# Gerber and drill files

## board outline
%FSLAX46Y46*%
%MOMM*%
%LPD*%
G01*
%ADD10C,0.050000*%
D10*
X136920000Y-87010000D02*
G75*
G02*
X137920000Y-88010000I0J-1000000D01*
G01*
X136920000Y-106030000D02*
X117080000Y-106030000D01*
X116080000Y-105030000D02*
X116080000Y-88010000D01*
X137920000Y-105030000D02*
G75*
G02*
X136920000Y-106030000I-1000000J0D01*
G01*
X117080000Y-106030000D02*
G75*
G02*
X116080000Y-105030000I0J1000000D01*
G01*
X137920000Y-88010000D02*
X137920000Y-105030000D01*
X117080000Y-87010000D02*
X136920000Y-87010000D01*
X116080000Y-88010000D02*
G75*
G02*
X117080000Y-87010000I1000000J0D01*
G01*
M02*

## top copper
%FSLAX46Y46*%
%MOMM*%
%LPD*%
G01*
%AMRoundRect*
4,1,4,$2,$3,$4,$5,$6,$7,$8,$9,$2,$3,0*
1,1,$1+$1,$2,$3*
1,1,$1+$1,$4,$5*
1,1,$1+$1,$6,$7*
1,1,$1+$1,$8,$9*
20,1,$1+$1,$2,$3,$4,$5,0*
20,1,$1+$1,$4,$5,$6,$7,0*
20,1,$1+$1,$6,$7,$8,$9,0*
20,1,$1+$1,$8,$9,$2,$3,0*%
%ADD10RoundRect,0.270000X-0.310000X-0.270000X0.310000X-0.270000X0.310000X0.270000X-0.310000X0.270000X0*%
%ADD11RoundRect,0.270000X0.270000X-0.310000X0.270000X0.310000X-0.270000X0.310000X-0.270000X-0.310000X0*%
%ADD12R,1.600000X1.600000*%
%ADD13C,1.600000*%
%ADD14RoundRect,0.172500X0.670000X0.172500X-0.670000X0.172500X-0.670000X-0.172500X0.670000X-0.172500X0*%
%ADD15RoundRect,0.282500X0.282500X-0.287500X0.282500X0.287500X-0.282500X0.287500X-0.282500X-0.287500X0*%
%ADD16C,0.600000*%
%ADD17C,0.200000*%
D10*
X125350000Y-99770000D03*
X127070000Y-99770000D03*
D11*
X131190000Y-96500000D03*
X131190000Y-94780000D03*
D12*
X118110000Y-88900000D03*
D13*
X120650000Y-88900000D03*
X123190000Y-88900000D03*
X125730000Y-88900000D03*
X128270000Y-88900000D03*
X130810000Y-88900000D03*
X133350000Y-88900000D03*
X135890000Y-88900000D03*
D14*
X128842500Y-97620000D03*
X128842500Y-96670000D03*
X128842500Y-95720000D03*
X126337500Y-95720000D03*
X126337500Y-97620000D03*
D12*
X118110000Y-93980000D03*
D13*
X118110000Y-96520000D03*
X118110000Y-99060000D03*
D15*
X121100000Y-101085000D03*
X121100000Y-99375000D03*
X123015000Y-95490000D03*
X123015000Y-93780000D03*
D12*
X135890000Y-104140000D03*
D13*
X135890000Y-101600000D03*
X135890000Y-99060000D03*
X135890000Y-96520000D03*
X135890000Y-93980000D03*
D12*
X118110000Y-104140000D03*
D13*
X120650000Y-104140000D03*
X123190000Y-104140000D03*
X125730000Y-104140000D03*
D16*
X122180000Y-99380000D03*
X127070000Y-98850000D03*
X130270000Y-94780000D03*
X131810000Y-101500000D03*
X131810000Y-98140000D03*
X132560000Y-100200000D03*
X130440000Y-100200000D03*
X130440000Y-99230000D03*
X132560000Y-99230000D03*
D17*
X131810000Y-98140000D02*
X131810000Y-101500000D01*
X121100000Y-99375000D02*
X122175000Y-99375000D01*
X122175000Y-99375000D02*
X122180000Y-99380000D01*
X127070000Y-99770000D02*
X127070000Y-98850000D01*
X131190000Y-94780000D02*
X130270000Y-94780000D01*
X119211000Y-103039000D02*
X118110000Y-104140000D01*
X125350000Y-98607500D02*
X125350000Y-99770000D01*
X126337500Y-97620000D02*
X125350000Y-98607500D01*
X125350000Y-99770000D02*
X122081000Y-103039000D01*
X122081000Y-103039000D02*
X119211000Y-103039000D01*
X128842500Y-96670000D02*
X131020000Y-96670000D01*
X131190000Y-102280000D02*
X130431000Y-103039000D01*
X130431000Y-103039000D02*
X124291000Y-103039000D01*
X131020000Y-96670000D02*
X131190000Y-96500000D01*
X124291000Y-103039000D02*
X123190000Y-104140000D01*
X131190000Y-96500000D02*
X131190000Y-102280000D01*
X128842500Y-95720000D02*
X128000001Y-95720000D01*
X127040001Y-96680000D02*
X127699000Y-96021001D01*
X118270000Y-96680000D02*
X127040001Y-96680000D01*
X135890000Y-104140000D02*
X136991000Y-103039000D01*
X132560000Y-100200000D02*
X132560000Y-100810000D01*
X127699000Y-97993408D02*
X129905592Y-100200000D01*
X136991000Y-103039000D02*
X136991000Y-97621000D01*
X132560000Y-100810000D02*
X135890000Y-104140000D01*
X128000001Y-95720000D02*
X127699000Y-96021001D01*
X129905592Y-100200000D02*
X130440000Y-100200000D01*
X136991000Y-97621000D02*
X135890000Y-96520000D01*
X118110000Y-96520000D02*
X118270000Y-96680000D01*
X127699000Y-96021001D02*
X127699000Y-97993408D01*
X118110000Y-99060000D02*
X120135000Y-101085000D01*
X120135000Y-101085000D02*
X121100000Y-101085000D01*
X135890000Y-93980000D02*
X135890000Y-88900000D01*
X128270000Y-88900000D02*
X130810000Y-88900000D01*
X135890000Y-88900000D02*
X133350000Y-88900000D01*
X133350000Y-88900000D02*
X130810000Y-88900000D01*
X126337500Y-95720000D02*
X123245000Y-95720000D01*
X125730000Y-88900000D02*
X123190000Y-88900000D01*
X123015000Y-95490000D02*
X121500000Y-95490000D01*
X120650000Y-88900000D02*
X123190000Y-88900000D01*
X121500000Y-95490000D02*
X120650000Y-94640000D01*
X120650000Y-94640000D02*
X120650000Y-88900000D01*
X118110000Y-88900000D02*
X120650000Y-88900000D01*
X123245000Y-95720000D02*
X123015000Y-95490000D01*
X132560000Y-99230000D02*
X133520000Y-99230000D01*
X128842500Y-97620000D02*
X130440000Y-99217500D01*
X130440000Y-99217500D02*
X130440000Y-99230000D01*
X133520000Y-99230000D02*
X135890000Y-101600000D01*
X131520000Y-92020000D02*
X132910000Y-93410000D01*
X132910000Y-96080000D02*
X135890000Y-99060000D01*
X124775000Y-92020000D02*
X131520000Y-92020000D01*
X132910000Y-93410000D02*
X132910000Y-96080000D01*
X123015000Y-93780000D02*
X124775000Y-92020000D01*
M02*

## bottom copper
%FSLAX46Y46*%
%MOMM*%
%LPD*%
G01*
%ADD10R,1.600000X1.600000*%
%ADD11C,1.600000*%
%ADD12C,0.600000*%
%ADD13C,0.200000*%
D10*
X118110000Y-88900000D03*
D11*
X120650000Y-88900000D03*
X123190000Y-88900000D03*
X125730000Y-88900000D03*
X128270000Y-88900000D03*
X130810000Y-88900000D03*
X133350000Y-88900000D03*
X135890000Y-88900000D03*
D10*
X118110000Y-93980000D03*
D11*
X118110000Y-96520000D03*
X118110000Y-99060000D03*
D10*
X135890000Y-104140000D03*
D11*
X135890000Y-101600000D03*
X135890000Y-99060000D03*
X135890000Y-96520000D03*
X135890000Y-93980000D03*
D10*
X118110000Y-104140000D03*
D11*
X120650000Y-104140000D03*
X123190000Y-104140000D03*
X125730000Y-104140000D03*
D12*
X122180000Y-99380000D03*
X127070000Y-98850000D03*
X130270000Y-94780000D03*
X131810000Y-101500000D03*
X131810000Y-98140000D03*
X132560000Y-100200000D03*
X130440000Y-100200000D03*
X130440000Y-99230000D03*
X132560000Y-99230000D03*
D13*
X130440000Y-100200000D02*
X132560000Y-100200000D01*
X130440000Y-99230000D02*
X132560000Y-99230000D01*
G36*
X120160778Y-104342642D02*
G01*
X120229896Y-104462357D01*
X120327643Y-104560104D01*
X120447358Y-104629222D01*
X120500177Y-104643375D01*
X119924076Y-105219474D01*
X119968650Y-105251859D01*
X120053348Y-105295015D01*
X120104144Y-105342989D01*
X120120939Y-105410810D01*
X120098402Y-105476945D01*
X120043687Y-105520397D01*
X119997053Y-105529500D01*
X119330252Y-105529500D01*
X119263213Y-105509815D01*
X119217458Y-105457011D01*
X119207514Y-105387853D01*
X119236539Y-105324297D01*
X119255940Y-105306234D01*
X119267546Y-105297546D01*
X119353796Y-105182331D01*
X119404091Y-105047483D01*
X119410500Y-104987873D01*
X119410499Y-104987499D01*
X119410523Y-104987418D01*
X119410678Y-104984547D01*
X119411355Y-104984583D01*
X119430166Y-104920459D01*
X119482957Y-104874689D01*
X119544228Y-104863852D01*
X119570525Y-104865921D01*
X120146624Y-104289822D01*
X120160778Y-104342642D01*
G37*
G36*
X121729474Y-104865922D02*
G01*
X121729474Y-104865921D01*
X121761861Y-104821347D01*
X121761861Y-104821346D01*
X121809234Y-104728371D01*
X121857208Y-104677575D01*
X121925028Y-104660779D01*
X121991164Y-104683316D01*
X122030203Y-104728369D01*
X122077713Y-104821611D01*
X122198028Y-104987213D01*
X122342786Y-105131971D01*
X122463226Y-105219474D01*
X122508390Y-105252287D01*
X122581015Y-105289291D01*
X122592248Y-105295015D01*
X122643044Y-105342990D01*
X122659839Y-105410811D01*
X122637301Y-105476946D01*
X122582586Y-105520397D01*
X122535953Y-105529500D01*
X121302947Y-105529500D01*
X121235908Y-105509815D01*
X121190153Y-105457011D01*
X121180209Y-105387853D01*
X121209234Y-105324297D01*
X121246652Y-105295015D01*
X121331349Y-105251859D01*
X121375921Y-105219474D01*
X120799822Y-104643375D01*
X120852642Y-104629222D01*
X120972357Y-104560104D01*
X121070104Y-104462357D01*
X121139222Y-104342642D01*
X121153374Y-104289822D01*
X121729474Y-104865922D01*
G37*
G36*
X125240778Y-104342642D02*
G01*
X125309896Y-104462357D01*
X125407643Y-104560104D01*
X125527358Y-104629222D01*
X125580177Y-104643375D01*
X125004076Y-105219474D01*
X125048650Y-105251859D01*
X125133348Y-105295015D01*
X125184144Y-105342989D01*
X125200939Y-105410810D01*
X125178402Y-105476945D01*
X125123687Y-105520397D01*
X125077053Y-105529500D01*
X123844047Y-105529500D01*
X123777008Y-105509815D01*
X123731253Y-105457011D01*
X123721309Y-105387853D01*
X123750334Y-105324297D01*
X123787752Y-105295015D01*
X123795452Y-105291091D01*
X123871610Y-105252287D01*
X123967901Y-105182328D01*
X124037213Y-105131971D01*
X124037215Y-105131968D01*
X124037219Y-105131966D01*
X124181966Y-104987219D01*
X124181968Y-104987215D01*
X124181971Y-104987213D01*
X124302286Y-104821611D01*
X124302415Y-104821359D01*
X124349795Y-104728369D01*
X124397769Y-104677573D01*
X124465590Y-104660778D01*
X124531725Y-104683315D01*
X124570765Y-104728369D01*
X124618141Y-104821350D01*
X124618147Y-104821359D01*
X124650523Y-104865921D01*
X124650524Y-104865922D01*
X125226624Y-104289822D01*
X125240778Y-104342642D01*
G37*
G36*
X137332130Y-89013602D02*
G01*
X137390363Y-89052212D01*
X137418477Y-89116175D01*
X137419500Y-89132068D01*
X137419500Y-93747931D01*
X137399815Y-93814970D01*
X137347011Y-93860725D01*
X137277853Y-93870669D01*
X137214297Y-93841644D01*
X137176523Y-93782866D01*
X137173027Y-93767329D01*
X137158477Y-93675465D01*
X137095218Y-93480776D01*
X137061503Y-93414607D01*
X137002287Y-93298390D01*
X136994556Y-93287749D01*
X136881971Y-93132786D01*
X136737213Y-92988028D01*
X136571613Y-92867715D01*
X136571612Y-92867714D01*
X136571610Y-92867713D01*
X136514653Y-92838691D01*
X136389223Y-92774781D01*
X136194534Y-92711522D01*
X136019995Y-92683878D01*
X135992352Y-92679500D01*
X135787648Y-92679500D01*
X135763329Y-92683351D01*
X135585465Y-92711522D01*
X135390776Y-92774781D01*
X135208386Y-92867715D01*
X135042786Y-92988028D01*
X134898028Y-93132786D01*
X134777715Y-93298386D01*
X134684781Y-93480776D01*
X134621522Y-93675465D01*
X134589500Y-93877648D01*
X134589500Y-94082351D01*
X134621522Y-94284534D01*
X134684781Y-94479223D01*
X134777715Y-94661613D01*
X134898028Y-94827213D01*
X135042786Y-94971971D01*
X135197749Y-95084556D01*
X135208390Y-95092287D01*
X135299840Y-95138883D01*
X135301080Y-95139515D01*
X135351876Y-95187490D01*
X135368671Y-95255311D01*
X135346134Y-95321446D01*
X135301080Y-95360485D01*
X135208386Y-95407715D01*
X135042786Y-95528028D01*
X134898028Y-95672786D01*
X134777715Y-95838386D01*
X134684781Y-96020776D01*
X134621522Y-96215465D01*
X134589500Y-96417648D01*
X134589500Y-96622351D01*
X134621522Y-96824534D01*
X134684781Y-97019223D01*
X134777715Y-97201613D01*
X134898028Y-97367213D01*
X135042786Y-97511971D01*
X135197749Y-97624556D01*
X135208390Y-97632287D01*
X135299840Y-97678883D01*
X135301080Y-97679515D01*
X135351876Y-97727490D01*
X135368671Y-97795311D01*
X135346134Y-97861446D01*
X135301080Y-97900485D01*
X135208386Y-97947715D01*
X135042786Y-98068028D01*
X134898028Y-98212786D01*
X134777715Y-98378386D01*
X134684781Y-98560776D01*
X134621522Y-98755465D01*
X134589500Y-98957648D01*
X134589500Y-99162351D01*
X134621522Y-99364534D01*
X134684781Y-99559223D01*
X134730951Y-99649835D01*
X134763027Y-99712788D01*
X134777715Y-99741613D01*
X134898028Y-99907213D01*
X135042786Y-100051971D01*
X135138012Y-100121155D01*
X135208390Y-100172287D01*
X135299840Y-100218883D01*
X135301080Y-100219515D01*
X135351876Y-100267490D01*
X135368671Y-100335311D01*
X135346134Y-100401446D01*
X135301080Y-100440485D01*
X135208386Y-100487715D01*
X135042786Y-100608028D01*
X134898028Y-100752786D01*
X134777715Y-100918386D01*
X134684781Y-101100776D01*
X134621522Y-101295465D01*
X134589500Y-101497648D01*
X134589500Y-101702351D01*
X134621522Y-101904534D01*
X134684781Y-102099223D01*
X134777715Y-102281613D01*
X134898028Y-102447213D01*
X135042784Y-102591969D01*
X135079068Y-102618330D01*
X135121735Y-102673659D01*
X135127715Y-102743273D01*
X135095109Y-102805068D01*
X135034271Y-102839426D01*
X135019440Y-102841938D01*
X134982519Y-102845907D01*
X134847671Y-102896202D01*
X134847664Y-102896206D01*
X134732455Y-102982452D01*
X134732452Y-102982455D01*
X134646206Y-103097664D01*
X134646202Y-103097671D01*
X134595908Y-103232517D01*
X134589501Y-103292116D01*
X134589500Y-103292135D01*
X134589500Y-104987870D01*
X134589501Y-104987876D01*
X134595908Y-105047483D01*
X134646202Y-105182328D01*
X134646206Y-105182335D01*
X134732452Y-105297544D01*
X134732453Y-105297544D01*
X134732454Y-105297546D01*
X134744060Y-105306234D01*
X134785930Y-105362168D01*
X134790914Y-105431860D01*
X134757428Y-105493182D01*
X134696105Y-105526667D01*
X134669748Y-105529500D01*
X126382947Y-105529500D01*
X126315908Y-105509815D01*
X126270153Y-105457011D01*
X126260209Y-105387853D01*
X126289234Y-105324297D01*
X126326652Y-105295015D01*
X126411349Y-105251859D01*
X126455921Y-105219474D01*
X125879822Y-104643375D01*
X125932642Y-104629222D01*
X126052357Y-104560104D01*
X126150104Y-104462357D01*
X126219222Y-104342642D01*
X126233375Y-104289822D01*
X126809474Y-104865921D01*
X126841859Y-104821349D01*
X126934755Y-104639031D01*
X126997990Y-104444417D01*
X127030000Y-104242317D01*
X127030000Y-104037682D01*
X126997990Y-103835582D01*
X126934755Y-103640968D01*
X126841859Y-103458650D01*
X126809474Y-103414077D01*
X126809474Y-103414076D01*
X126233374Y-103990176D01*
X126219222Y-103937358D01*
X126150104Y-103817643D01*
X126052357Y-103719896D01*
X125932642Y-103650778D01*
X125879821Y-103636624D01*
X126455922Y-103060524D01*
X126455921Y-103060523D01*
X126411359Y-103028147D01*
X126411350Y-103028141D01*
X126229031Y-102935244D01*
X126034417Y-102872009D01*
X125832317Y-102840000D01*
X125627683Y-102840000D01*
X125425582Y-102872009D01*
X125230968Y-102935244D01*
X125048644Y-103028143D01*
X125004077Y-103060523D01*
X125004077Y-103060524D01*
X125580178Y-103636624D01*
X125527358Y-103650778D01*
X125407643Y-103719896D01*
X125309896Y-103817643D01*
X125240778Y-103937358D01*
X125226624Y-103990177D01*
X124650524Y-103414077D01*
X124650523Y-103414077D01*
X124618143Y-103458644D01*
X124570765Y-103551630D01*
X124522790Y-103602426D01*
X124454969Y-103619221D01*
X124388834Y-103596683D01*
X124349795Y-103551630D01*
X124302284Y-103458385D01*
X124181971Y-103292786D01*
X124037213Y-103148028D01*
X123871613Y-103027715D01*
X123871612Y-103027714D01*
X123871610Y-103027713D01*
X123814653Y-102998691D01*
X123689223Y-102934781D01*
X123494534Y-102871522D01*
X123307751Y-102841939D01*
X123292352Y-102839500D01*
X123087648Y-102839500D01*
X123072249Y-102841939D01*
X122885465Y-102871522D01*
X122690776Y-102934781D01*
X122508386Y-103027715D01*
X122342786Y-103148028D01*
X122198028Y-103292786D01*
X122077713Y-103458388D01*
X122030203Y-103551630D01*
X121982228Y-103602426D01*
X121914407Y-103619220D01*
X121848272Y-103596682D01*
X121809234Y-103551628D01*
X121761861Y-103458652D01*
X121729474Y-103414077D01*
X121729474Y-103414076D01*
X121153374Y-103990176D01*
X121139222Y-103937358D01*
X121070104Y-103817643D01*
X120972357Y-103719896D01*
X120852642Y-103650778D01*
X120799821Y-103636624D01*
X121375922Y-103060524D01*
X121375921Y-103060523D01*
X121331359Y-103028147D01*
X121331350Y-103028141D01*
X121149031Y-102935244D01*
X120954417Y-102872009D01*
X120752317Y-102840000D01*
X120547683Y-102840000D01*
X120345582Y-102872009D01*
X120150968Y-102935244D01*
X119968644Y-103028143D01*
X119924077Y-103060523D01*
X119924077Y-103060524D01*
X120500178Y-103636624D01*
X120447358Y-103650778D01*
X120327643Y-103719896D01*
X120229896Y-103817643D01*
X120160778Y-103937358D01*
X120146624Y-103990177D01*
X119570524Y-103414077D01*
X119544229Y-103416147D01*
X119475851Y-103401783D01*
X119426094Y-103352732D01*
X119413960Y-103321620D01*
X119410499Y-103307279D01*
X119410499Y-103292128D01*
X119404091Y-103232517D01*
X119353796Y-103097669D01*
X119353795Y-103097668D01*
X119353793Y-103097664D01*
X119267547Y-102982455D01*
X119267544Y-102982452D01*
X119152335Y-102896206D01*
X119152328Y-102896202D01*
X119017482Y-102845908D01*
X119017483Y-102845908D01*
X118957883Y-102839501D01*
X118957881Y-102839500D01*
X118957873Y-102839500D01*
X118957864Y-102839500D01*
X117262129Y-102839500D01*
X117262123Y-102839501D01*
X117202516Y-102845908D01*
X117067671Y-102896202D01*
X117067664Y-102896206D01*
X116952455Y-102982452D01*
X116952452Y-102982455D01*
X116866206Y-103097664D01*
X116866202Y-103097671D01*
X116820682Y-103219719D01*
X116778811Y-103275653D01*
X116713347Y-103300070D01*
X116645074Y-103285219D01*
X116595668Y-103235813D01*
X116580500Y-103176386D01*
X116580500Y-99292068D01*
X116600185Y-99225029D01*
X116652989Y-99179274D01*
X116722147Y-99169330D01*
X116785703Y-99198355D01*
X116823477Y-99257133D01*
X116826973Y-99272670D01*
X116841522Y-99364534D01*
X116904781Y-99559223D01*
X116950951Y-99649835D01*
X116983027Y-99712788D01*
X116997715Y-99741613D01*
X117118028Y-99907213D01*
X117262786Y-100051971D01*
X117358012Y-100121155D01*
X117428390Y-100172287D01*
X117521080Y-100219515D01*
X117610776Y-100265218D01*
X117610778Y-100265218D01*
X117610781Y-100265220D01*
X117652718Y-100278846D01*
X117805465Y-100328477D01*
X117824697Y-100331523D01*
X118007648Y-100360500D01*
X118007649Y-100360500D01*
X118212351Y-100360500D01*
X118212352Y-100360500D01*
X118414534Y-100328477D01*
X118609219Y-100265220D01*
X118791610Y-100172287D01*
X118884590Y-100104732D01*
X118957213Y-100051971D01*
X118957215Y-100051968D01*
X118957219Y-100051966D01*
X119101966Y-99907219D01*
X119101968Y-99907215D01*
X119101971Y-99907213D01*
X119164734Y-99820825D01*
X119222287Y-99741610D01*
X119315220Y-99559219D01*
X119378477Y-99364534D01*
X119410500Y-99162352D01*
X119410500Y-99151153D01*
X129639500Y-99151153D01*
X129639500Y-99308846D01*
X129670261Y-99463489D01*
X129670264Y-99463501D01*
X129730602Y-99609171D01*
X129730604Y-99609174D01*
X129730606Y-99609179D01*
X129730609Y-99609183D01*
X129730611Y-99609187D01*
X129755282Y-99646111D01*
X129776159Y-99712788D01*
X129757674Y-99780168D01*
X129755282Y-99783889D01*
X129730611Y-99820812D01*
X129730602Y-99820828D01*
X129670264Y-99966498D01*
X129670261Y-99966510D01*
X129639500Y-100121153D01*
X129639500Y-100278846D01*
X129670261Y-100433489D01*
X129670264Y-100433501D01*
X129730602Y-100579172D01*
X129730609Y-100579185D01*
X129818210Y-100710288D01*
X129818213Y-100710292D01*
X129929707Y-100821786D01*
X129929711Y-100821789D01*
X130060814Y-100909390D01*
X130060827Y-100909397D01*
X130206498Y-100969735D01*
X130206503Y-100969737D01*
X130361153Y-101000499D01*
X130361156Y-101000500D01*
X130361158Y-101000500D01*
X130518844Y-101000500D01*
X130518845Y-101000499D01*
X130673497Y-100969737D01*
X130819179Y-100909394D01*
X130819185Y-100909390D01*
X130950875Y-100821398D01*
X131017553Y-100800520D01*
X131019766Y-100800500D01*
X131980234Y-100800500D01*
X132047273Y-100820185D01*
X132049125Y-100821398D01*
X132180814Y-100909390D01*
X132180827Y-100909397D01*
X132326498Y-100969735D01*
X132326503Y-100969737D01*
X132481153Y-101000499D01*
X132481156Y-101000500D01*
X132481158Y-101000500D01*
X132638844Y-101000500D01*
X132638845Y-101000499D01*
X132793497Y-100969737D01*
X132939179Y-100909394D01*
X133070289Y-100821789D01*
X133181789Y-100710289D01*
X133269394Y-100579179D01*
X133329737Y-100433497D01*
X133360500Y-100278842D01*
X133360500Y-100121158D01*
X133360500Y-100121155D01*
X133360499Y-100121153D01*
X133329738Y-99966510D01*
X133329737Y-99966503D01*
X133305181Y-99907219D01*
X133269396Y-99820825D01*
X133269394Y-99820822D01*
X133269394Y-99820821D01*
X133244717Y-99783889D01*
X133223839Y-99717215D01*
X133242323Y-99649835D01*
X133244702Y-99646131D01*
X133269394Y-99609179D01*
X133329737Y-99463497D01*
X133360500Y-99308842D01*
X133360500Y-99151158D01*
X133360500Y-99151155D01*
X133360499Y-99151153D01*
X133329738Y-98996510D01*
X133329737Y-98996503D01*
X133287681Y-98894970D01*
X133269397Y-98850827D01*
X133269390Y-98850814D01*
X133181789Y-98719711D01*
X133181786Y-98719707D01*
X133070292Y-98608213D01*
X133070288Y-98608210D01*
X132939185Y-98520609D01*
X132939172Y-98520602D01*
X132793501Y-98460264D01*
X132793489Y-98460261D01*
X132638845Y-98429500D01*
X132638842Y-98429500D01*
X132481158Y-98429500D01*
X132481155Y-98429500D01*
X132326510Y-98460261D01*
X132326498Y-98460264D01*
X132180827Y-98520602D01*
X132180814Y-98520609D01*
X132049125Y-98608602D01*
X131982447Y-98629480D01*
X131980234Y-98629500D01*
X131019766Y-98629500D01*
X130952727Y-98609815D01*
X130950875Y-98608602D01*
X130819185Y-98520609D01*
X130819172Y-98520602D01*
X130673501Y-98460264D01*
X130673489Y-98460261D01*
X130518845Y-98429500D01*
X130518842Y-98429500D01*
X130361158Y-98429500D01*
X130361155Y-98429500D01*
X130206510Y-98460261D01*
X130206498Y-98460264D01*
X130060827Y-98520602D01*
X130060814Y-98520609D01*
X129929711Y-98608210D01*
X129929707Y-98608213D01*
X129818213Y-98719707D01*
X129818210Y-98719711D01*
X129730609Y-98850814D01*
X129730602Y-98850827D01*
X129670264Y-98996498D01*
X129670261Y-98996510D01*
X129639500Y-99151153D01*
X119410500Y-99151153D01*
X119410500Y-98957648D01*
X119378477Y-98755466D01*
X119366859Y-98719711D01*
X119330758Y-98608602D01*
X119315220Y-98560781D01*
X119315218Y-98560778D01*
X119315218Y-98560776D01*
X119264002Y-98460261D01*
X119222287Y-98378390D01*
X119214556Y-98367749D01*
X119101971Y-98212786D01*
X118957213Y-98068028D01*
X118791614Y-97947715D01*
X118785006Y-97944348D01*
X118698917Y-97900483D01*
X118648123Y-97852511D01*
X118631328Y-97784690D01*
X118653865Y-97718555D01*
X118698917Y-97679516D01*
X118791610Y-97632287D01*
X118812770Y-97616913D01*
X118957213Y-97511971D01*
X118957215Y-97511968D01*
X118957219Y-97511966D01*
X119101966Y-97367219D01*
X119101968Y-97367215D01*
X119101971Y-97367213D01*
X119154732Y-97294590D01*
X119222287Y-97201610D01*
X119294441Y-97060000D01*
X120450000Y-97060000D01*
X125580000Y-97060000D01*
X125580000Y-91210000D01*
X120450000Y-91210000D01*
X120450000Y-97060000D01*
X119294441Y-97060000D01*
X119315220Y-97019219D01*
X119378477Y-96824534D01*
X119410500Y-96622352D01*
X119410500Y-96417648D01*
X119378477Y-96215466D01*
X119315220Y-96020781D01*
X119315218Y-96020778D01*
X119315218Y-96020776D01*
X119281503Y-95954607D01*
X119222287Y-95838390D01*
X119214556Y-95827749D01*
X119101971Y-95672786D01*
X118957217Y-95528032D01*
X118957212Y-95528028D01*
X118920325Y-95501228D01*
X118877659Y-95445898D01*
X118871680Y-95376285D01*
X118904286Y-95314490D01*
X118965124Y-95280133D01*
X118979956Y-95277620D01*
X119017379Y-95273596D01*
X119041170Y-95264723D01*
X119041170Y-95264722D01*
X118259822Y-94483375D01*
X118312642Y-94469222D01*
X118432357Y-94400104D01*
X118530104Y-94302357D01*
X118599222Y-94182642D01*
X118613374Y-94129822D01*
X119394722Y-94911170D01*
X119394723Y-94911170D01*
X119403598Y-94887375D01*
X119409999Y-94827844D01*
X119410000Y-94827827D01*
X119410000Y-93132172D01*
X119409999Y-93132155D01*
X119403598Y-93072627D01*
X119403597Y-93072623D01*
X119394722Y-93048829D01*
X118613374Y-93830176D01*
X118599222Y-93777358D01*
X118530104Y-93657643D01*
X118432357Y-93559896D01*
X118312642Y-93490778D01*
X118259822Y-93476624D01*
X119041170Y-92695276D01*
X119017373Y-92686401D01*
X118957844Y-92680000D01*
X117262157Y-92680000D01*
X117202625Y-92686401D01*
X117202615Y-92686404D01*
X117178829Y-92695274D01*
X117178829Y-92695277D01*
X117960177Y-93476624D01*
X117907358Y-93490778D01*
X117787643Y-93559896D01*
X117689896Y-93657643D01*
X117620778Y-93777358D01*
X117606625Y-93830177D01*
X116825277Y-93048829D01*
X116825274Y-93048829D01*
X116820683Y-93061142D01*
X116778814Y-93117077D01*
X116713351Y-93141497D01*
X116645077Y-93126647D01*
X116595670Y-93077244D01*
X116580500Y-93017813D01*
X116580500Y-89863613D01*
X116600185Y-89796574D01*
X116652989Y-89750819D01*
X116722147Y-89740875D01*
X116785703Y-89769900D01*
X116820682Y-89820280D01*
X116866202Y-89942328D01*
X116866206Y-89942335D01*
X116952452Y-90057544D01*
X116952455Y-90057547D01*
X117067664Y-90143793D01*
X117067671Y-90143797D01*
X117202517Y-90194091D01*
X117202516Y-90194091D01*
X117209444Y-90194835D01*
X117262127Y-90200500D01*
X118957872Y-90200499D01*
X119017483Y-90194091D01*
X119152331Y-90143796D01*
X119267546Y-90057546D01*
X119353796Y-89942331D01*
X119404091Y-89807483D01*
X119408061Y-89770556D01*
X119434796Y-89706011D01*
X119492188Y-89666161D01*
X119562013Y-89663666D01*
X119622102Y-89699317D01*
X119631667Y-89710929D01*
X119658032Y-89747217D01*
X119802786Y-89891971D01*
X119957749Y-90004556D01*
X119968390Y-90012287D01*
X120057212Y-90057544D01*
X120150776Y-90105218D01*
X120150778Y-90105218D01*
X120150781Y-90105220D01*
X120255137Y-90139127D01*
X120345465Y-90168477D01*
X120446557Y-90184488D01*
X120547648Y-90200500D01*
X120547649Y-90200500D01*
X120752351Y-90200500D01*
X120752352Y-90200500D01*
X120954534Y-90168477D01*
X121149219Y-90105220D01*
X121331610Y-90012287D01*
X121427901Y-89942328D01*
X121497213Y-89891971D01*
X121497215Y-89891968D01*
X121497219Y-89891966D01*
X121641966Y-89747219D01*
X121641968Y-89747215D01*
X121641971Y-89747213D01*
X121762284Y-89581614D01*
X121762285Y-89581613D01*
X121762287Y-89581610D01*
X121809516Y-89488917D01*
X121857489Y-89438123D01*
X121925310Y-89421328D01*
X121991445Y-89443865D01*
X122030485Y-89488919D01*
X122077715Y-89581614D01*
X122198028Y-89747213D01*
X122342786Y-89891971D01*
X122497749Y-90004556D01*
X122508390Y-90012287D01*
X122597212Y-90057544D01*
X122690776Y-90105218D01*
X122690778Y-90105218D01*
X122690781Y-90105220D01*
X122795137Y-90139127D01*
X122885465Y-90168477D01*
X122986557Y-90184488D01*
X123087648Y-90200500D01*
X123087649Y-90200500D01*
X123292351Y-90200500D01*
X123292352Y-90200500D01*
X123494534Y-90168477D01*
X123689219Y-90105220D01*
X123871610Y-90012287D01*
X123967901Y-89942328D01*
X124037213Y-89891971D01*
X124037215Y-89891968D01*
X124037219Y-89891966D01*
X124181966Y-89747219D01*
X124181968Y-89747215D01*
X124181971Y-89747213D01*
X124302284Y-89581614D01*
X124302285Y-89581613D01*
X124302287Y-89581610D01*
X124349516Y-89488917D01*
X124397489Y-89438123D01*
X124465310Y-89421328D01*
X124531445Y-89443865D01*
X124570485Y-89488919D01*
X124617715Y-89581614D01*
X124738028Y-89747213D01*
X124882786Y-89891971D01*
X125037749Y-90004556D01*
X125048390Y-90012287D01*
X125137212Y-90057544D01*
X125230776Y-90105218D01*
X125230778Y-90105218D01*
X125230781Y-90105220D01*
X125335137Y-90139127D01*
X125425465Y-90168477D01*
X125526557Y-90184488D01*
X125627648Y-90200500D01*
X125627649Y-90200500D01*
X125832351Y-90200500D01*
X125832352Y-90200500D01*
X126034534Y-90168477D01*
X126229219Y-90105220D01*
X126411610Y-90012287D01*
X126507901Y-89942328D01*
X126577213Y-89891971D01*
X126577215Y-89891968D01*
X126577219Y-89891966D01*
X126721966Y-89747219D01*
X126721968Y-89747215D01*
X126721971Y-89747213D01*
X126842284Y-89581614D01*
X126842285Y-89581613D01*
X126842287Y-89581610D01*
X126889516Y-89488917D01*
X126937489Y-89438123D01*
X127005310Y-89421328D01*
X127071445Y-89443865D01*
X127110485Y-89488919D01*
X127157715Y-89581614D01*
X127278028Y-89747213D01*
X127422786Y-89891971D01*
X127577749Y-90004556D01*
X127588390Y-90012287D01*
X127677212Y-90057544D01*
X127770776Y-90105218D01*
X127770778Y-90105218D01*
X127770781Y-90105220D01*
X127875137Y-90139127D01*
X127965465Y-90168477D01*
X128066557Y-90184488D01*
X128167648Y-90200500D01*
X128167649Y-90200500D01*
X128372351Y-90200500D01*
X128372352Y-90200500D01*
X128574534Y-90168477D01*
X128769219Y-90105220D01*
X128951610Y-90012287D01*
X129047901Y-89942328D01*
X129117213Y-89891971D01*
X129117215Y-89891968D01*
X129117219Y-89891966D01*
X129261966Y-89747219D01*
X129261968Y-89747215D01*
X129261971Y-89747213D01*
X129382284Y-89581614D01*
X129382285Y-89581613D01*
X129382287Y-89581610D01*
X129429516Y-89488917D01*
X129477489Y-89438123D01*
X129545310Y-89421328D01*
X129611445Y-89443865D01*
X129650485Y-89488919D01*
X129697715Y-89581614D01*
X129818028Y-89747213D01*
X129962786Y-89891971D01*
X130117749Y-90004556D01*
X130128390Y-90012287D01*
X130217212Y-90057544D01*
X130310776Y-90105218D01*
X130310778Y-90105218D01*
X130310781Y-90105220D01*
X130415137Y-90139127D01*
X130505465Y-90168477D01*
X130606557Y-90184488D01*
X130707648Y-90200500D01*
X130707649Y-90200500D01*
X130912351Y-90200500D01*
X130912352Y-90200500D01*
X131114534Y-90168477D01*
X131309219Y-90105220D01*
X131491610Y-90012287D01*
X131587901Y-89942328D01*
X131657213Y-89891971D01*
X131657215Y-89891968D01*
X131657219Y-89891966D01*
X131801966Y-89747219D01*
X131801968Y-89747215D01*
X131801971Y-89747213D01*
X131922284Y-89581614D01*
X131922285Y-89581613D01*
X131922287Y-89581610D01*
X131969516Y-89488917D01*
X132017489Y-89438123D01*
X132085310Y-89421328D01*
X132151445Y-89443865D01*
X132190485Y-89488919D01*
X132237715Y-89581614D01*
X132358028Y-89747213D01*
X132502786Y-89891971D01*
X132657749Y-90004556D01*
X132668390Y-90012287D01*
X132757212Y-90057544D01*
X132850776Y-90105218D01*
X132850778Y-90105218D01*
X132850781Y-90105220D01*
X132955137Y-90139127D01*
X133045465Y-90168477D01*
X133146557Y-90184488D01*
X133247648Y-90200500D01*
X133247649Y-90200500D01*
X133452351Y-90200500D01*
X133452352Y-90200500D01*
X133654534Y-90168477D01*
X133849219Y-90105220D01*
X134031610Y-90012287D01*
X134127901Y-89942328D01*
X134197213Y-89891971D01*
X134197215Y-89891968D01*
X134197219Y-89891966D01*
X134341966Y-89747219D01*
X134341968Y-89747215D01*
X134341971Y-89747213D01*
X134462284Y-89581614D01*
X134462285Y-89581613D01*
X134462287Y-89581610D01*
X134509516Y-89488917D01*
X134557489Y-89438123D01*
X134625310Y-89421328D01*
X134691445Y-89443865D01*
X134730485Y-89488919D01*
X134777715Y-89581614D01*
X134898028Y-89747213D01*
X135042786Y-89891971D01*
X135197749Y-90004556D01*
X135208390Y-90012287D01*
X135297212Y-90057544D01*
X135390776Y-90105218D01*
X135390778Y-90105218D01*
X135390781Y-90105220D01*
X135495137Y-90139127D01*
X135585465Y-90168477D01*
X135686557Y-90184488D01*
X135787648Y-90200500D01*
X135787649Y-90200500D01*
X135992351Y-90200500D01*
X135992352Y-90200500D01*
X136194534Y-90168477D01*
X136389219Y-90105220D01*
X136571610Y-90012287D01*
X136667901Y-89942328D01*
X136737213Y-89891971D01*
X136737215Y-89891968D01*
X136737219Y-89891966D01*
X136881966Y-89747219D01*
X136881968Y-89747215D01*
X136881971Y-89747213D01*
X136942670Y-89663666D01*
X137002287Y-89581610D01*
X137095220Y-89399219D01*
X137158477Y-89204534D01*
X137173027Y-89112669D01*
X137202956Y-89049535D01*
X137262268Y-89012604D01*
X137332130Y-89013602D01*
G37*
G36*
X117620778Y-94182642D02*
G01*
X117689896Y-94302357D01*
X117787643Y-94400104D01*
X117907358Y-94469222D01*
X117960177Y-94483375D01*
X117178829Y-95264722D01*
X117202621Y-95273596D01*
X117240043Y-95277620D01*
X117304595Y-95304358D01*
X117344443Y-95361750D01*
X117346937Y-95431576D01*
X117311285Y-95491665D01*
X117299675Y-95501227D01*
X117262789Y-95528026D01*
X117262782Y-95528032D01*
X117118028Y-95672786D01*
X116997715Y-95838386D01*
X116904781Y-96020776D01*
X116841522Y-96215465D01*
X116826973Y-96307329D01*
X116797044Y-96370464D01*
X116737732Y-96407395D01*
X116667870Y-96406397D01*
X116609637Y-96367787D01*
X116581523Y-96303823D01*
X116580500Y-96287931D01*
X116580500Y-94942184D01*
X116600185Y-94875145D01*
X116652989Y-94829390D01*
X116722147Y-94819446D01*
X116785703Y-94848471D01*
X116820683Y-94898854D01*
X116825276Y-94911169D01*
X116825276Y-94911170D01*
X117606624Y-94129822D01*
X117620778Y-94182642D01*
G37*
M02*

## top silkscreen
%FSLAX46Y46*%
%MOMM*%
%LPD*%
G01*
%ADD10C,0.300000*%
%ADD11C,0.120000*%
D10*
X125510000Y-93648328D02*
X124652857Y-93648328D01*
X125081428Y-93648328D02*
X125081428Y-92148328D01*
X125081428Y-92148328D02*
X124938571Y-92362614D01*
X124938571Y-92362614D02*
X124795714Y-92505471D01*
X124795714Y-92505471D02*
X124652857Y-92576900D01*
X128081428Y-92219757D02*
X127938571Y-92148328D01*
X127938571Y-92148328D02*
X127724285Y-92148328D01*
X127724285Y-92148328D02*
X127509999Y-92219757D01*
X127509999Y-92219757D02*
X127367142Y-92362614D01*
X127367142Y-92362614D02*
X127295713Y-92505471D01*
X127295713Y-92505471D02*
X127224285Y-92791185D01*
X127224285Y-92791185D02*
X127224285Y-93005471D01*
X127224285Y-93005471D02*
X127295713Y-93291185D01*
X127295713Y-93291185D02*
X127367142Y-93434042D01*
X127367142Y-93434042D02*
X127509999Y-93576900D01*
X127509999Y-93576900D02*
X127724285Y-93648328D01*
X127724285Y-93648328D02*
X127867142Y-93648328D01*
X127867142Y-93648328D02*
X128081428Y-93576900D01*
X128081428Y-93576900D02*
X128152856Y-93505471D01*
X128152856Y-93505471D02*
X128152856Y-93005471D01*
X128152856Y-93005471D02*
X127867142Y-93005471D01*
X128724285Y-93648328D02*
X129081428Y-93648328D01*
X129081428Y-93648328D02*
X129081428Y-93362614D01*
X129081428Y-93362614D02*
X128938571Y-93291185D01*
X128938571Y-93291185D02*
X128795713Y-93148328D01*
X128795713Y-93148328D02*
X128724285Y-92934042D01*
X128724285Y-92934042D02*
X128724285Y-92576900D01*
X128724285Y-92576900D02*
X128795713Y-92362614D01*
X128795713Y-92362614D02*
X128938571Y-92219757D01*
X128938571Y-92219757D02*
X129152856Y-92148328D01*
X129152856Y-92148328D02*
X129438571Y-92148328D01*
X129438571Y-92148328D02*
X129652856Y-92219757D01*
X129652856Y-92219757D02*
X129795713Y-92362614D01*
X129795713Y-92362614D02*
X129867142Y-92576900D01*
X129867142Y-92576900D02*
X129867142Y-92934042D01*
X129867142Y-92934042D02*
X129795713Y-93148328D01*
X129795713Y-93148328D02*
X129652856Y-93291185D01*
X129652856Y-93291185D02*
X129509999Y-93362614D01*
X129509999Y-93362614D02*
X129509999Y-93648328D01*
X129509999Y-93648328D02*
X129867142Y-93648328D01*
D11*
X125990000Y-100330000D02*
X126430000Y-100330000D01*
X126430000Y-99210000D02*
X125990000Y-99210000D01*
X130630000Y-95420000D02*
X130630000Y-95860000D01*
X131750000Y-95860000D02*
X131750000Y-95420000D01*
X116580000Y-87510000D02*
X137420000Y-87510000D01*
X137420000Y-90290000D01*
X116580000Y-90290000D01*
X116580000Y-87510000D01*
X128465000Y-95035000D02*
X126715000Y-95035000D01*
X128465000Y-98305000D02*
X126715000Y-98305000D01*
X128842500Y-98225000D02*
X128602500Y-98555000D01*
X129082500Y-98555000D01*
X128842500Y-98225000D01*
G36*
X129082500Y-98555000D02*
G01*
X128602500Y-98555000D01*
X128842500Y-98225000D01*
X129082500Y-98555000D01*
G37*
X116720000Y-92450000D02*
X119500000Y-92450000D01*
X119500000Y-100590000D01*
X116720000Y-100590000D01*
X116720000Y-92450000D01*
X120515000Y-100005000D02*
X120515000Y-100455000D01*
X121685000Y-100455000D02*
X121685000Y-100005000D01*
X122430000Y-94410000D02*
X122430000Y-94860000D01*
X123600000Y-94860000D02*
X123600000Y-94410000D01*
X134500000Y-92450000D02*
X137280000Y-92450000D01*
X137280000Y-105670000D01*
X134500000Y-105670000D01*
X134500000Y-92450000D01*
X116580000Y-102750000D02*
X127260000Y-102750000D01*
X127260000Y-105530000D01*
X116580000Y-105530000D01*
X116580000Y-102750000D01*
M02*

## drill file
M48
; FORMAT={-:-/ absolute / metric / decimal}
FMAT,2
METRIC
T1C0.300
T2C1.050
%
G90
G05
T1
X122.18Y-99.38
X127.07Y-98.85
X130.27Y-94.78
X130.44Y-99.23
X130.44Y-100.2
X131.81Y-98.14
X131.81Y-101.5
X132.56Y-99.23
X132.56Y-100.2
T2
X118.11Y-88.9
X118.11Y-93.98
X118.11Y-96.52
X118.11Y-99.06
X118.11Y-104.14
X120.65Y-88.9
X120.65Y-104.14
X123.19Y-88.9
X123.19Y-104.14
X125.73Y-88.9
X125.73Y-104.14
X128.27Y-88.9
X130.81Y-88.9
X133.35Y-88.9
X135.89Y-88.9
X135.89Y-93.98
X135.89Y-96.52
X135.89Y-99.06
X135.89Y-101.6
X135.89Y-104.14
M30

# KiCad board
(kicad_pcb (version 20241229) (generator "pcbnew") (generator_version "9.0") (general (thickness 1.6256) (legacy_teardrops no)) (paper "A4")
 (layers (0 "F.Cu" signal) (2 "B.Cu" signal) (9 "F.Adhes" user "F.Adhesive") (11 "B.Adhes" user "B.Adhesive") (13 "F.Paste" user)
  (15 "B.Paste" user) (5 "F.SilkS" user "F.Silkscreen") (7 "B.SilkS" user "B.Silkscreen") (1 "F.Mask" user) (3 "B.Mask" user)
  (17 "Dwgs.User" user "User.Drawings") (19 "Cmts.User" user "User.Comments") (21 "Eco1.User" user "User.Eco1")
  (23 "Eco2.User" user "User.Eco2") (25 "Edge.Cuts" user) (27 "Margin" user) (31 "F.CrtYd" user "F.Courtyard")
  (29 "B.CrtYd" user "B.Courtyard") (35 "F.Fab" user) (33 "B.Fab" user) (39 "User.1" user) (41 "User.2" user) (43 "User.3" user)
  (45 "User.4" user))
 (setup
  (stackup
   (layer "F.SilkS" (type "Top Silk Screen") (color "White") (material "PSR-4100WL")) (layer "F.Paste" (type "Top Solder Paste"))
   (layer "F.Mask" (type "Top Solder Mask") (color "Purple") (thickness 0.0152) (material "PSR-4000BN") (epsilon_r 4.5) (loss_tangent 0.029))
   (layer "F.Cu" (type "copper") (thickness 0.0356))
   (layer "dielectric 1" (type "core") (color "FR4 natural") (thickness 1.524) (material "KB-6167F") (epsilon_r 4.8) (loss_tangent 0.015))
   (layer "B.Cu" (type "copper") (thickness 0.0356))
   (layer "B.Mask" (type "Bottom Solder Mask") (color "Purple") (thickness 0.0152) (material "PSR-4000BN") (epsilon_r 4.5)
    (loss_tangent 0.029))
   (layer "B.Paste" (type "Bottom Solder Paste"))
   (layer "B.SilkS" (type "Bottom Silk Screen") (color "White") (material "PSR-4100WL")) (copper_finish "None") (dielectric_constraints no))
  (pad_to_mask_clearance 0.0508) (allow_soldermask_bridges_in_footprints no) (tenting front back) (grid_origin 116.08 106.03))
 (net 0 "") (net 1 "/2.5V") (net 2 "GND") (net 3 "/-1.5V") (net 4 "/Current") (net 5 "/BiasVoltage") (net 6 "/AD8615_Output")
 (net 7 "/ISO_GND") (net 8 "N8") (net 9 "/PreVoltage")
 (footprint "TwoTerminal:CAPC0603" (layer "F.Cu") (at 126.21 99.77)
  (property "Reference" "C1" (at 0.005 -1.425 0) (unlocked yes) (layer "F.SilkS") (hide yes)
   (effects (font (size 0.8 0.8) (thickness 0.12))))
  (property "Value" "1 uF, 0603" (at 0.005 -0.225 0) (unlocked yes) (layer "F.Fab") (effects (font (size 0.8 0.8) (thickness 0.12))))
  (fp_line (start -0.22 0.56) (end 0.22 0.56) (stroke (width 0.12) (type default)) (layer "F.SilkS"))
  (fp_line (start 0.22 -0.56) (end -0.22 -0.56) (stroke (width 0.12) (type default)) (layer "F.SilkS"))
  (pad "1" smd roundrect (at -0.86 0) (size 1.16 1.08) (layers "F.Cu" "F.Mask" "F.Paste") (roundrect_rratio 0.25) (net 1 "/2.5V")
   (thermal_bridge_angle 45))
  (pad "2" smd roundrect (at 0.86 0) (size 1.16 1.08) (layers "F.Cu" "F.Mask" "F.Paste") (roundrect_rratio 0.25) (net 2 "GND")
   (thermal_bridge_angle 45)))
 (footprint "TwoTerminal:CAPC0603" (layer "F.Cu") (at 131.19 95.64 90)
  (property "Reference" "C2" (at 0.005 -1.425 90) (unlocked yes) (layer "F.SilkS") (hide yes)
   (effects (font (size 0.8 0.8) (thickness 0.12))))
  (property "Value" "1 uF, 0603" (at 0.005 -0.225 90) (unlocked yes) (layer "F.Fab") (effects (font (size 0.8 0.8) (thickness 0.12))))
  (fp_line (start 0.22 -0.56) (end -0.22 -0.56) (stroke (width 0.12) (type default)) (layer "F.SilkS"))
  (fp_line (start -0.22 0.56) (end 0.22 0.56) (stroke (width 0.12) (type default)) (layer "F.SilkS"))
  (pad "1" smd roundrect (at -0.86 0 90) (size 1.16 1.08) (layers "F.Cu" "F.Mask" "F.Paste") (roundrect_rratio 0.25) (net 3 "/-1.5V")
   (thermal_bridge_angle 45))
  (pad "2" smd roundrect (at 0.86 0 90) (size 1.16 1.08) (layers "F.Cu" "F.Mask" "F.Paste") (roundrect_rratio 0.25) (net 2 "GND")
   (thermal_bridge_angle 45)))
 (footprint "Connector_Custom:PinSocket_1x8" (layer "F.Cu") (at 127 88.9 90)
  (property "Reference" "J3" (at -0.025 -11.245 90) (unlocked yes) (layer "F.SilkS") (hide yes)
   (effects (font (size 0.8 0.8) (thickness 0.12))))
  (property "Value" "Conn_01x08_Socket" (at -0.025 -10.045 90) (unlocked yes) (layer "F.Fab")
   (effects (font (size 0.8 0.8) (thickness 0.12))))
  (fp_rect (start -1.39 -10.42) (end 1.39 10.42) (stroke (width 0.12) (type default)) (fill no) (layer "F.SilkS"))
  (pad "1" thru_hole rect (at 0 -8.89 90) (size 1.6 1.6) (drill 1.05) (layers "*.Cu" "*.Mask") (remove_unused_layers no) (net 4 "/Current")
   (thermal_bridge_angle 45))
  (pad "2" thru_hole circle (at 0 -6.35 90) (size 1.6 1.6) (drill 1.05) (layers "*.Cu" "*.Mask") (remove_unused_layers no)
   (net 4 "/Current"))
  (pad "3" thru_hole circle (at 0 -3.81 90) (size 1.6 1.6) (drill 1.05) (layers "*.Cu" "*.Mask") (remove_unused_layers no)
   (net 4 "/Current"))
  (pad "4" thru_hole circle (at 0 -1.27 90) (size 1.6 1.6) (drill 1.05) (layers "*.Cu" "*.Mask") (remove_unused_layers no)
   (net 4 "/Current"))
  (pad "5" thru_hole circle (at 0 1.27 90) (size 1.6 1.6) (drill 1.05) (layers "*.Cu" "*.Mask") (remove_unused_layers no)
   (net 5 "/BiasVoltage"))
  (pad "6" thru_hole circle (at 0 3.81 90) (size 1.6 1.6) (drill 1.05) (layers "*.Cu" "*.Mask") (remove_unused_layers no)
   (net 5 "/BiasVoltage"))
  (pad "7" thru_hole circle (at 0 6.35 90) (size 1.6 1.6) (drill 1.05) (layers "*.Cu" "*.Mask") (remove_unused_layers no)
   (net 5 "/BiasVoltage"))
  (pad "8" thru_hole circle (at 0 8.89 90) (size 1.6 1.6) (drill 1.05) (layers "*.Cu" "*.Mask") (remove_unused_layers no)
   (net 5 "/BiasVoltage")))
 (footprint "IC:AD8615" (layer "F.Cu") (at 127.59 96.67 180)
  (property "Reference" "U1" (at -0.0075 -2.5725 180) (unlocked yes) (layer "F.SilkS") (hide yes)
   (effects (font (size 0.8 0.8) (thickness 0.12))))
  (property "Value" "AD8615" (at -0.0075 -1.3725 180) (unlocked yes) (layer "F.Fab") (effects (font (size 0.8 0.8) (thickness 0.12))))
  (fp_line (start -0.875 1.635) (end 0.875 1.635) (stroke (width 0.12) (type default)) (layer "F.SilkS"))
  (fp_line (start -0.875 -1.635) (end 0.875 -1.635) (stroke (width 0.12) (type default)) (layer "F.SilkS"))
  (fp_poly
   (pts (xy -1.2525 -1.555) (xy -1.0125 -1.885) (xy -1.4925 -1.885)) (stroke (width 0.12) (type solid)) (fill yes) (layer "F.SilkS"))
  (pad "1" smd roundrect (at -1.2525 -0.95 180) (size 1.685 0.69) (layers "F.Cu" "F.Mask" "F.Paste") (roundrect_rratio 0.25)
   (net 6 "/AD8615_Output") (thermal_bridge_angle 45))
  (pad "2" smd roundrect (at -1.2525 0 180) (size 1.685 0.69) (layers "F.Cu" "F.Mask" "F.Paste") (roundrect_rratio 0.25) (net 3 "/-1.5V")
   (thermal_bridge_angle 45))
  (pad "3" smd roundrect (at -1.2525 0.95 180) (size 1.685 0.69) (layers "F.Cu" "F.Mask" "F.Paste") (roundrect_rratio 0.25)
   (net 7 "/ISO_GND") (thermal_bridge_angle 45))
  (pad "4" smd roundrect (at 1.2525 0.95 180) (size 1.685 0.69) (layers "F.Cu" "F.Mask" "F.Paste") (roundrect_rratio 0.25)
   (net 4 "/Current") (thermal_bridge_angle 45))
  (pad "5" smd roundrect (at 1.2525 -0.95 180) (size 1.685 0.69) (layers "F.Cu" "F.Mask" "F.Paste") (roundrect_rratio 0.25) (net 1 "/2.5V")
   (thermal_bridge_angle 45)))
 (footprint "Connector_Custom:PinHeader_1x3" (layer "F.Cu") (at 118.11 96.52)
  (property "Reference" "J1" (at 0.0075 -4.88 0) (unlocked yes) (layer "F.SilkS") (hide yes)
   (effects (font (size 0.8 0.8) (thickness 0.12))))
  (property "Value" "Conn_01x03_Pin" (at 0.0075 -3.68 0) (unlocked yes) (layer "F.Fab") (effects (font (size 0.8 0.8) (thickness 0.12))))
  (fp_rect (start -1.39 -4.07) (end 1.39 4.07) (stroke (width 0.12) (type default)) (fill no) (layer "F.SilkS"))
  (pad "1" thru_hole rect (at 0 -2.54) (size 1.6 1.6) (drill 1.05) (layers "*.Cu" "*.Mask") (remove_unused_layers no) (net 2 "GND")
   (thermal_bridge_angle 45))
  (pad "2" thru_hole circle (at 0 0) (size 1.6 1.6) (drill 1.05) (layers "*.Cu" "*.Mask") (remove_unused_layers no) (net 7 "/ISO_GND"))
  (pad "3" thru_hole circle (at 0 2.54) (size 1.6 1.6) (drill 1.05) (layers "*.Cu" "*.Mask") (remove_unused_layers no) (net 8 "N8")))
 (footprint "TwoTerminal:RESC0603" (layer "F.Cu") (at 121.1 100.23 90)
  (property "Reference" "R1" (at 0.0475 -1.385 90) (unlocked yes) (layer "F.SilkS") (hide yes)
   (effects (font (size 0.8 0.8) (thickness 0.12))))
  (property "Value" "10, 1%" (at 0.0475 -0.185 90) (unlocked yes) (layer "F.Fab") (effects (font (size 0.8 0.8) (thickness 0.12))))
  (fp_line (start 0.225 -0.585) (end -0.225 -0.585) (stroke (width 0.12) (type default)) (layer "F.SilkS"))
  (fp_line (start -0.225 0.585) (end 0.225 0.585) (stroke (width 0.12) (type default)) (layer "F.SilkS"))
  (pad "1" smd roundrect (at -0.855 0 90) (size 1.14 1.13) (layers "F.Cu" "F.Mask" "F.Paste") (roundrect_rratio 0.25) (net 8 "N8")
   (thermal_bridge_angle 45))
  (pad "2" smd roundrect (at 0.855 0 90) (size 1.14 1.13) (layers "F.Cu" "F.Mask" "F.Paste") (roundrect_rratio 0.25) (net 2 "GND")
   (thermal_bridge_angle 45)))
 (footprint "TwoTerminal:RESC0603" (layer "F.Cu") (at 123.015 94.635 90)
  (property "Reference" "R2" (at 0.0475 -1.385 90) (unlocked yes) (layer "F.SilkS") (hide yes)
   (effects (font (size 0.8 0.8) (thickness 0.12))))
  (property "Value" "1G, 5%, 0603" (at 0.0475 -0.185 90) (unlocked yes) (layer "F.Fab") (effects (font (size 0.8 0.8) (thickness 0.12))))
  (fp_line (start 0.225 -0.585) (end -0.225 -0.585) (stroke (width 0.12) (type default)) (layer "F.SilkS"))
  (fp_line (start -0.225 0.585) (end 0.225 0.585) (stroke (width 0.12) (type default)) (layer "F.SilkS"))
  (pad "1" smd roundrect (at -0.855 0 90) (size 1.14 1.13) (layers "F.Cu" "F.Mask" "F.Paste") (roundrect_rratio 0.25) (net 4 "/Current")
   (thermal_bridge_angle 45))
  (pad "2" smd roundrect (at 0.855 0 90) (size 1.14 1.13) (layers "F.Cu" "F.Mask" "F.Paste") (roundrect_rratio 0.25) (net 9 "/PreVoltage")
   (thermal_bridge_angle 45)))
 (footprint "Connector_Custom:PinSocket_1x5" (layer "F.Cu") (at 135.89 99.06 180)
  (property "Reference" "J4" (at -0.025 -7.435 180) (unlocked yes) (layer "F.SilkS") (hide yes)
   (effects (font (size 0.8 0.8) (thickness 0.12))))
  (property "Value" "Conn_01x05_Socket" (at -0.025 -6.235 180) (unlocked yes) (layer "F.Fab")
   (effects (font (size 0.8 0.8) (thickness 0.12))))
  (fp_rect (start -1.39 -6.61) (end 1.39 6.61) (stroke (width 0.12) (type default)) (fill no) (layer "F.SilkS"))
  (pad "1" thru_hole rect (at 0 -5.08 180) (size 1.6 1.6) (drill 1.05) (layers "*.Cu" "*.Mask") (remove_unused_layers no) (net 7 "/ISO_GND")
   (thermal_bridge_angle 45))
  (pad "2" thru_hole circle (at 0 -2.54 180) (size 1.6 1.6) (drill 1.05) (layers "*.Cu" "*.Mask") (remove_unused_layers no)
   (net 6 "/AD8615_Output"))
  (pad "3" thru_hole circle (at 0 0 180) (size 1.6 1.6) (drill 1.05) (layers "*.Cu" "*.Mask") (remove_unused_layers no)
   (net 9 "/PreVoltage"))
  (pad "4" thru_hole circle (at 0 2.54 180) (size 1.6 1.6) (drill 1.05) (layers "*.Cu" "*.Mask") (remove_unused_layers no)
   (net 7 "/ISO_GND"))
  (pad "5" thru_hole circle (at 0 5.08 180) (size 1.6 1.6) (drill 1.05) (layers "*.Cu" "*.Mask") (remove_unused_layers no)
   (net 5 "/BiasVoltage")))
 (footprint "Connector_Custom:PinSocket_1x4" (layer "F.Cu") (at 121.92 104.14 90)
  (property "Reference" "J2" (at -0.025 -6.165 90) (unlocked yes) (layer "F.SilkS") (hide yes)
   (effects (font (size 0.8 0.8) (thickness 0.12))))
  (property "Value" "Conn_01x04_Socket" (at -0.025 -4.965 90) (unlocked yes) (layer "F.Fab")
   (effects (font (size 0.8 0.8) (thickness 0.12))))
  (fp_rect (start -1.39 -5.34) (end 1.39 5.34) (stroke (width 0.12) (type default)) (fill no) (layer "F.SilkS"))
  (pad "1" thru_hole rect (at 0 -3.81 90) (size 1.6 1.6) (drill 1.05) (layers "*.Cu" "*.Mask") (remove_unused_layers no) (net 1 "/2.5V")
   (thermal_bridge_angle 45))
  (pad "2" thru_hole circle (at 0 -1.27 90) (size 1.6 1.6) (drill 1.05) (layers "*.Cu" "*.Mask") (remove_unused_layers no) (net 2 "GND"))
  (pad "3" thru_hole circle (at 0 1.27 90) (size 1.6 1.6) (drill 1.05) (layers "*.Cu" "*.Mask") (remove_unused_layers no) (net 3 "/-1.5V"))
  (pad "4" thru_hole circle (at 0 3.81 90) (size 1.6 1.6) (drill 1.05) (layers "*.Cu" "*.Mask") (remove_unused_layers no) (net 2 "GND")))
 (gr_arc (start 136.92 87.01) (mid 137.627107 87.302893) (end 137.92 88.01) (stroke (width 0.05) (type default)) (layer "Edge.Cuts"))
 (gr_line (start 136.92 106.03) (end 117.08 106.03) (stroke (width 0.05) (type default)) (layer "Edge.Cuts"))
 (gr_line (start 116.08 105.03) (end 116.08 88.01) (stroke (width 0.05) (type default)) (layer "Edge.Cuts"))
 (gr_arc (start 137.92 105.03) (mid 137.627107 105.737107) (end 136.92 106.03) (stroke (width 0.05) (type default)) (layer "Edge.Cuts"))
 (gr_arc (start 117.08 106.03) (mid 116.372893 105.737107) (end 116.08 105.03) (stroke (width 0.05) (type default)) (layer "Edge.Cuts"))
 (gr_line (start 137.92 88.01) (end 137.92 105.03) (stroke (width 0.05) (type default)) (layer "Edge.Cuts"))
 (gr_line (start 117.08 87.01) (end 136.92 87.01) (stroke (width 0.05) (type default)) (layer "Edge.Cuts"))
 (gr_arc (start 116.08 88.01) (mid 116.372893 87.302893) (end 117.08 87.01) (stroke (width 0.05) (type default)) (layer "Edge.Cuts"))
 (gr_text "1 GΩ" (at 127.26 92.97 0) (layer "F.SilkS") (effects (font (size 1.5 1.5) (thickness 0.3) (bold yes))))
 (segment (start 131.81 98.14) (end 131.81 101.5) (width 0.2) (layer "F.Cu") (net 2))
 (segment (start 121.1 99.375) (end 122.175 99.375) (width 0.2) (layer "F.Cu") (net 2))
 (segment (start 122.175 99.375) (end 122.18 99.38) (width 0.2) (layer "F.Cu") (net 2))
 (segment (start 127.07 99.77) (end 127.07 98.85) (width 0.2) (layer "F.Cu") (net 2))
 (segment (start 131.19 94.78) (end 130.27 94.78) (width 0.2) (layer "F.Cu") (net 2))
 (via (at 122.18 99.38) (size 0.6) (drill 0.3) (layers "F.Cu" "B.Cu") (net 2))
 (via (at 127.07 98.85) (size 0.6) (drill 0.3) (layers "F.Cu" "B.Cu") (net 2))
 (via (at 130.27 94.78) (size 0.6) (drill 0.3) (layers "F.Cu" "B.Cu") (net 2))
 (via (at 131.81 101.5) (size 0.6) (drill 0.3) (layers "F.Cu" "B.Cu") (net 2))
 (via (at 131.81 98.14) (size 0.6) (drill 0.3) (layers "F.Cu" "B.Cu") (free yes) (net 2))
 (segment (start 119.211 103.039) (end 118.11 104.14) (width 0.2) (layer "F.Cu") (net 1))
 (segment (start 125.35 98.6075) (end 125.35 99.77) (width 0.2) (layer "F.Cu") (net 1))
 (segment (start 126.3375 97.62) (end 125.35 98.6075) (width 0.2) (layer "F.Cu") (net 1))
 (segment (start 125.35 99.77) (end 122.081 103.039) (width 0.2) (layer "F.Cu") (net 1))
 (segment (start 122.081 103.039) (end 119.211 103.039) (width 0.2) (layer "F.Cu") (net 1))
 (segment (start 128.8425 96.67) (end 131.02 96.67) (width 0.2) (layer "F.Cu") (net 3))
 (segment (start 131.19 102.28) (end 130.431 103.039) (width 0.2) (layer "F.Cu") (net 3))
 (segment (start 130.431 103.039) (end 124.291 103.039) (width 0.2) (layer "F.Cu") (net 3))
 (segment (start 131.02 96.67) (end 131.19 96.5) (width 0.2) (layer "F.Cu") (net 3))
 (segment (start 124.291 103.039) (end 123.19 104.14) (width 0.2) (layer "F.Cu") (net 3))
 (segment (start 131.19 96.5) (end 131.19 102.28) (width 0.2) (layer "F.Cu") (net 3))
 (segment (start 128.8425 95.72) (end 128.000001 95.72) (width 0.2) (layer "F.Cu") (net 7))
 (segment (start 127.040001 96.68) (end 127.699 96.021001) (width 0.2) (layer "F.Cu") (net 7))
 (segment (start 118.27 96.68) (end 127.040001 96.68) (width 0.2) (layer "F.Cu") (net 7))
 (segment (start 135.89 104.14) (end 136.991 103.039) (width 0.2) (layer "F.Cu") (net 7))
 (segment (start 132.56 100.2) (end 132.56 100.81) (width 0.2) (layer "F.Cu") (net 7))
 (segment (start 127.699 97.993408) (end 129.905592 100.2) (width 0.2) (layer "F.Cu") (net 7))
 (segment (start 136.991 103.039) (end 136.991 97.621) (width 0.2) (layer "F.Cu") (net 7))
 (segment (start 132.56 100.81) (end 135.89 104.14) (width 0.2) (layer "F.Cu") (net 7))
 (segment (start 128.000001 95.72) (end 127.699 96.021001) (width 0.2) (layer "F.Cu") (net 7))
 (segment (start 129.905592 100.2) (end 130.44 100.2) (width 0.2) (layer "F.Cu") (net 7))
 (segment (start 136.991 97.621) (end 135.89 96.52) (width 0.2) (layer "F.Cu") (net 7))
 (segment (start 118.11 96.52) (end 118.27 96.68) (width 0.2) (layer "F.Cu") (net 7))
 (segment (start 127.699 96.021001) (end 127.699 97.993408) (width 0.2) (layer "F.Cu") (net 7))
 (via (at 132.56 100.2) (size 0.6) (drill 0.3) (layers "F.Cu" "B.Cu") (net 7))
 (via (at 130.44 100.2) (size 0.6) (drill 0.3) (layers "F.Cu" "B.Cu") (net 7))
 (segment (start 130.44 100.2) (end 132.56 100.2) (width 0.2) (layer "B.Cu") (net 7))
 (segment (start 118.11 99.06) (end 120.135 101.085) (width 0.2) (layer "F.Cu") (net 8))
 (segment (start 120.135 101.085) (end 121.1 101.085) (width 0.2) (layer "F.Cu") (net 8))
 (segment (start 135.89 93.98) (end 135.89 88.9) (width 0.2) (layer "F.Cu") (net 5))
 (segment (start 128.27 88.9) (end 130.81 88.9) (width 0.2) (layer "F.Cu") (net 5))
 (segment (start 135.89 88.9) (end 133.35 88.9) (width 0.2) (layer "F.Cu") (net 5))
 (segment (start 133.35 88.9) (end 130.81 88.9) (width 0.2) (layer "F.Cu") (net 5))
 (segment (start 126.3375 95.72) (end 123.245 95.72) (width 0.2) (layer "F.Cu") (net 4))
 (segment (start 125.73 88.9) (end 123.19 88.9) (width 0.2) (layer "F.Cu") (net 4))
 (segment (start 123.015 95.49) (end 121.5 95.49) (width 0.2) (layer "F.Cu") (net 4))
 (segment (start 120.65 88.9) (end 123.19 88.9) (width 0.2) (layer "F.Cu") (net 4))
 (segment (start 121.5 95.49) (end 120.65 94.64) (width 0.2) (layer "F.Cu") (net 4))
 (segment (start 120.65 94.64) (end 120.65 88.9) (width 0.2) (layer "F.Cu") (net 4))
 (segment (start 118.11 88.9) (end 120.65 88.9) (width 0.2) (layer "F.Cu") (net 4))
 (segment (start 123.245 95.72) (end 123.015 95.49) (width 0.2) (layer "F.Cu") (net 4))
 (segment (start 132.56 99.23) (end 133.52 99.23) (width 0.2) (layer "F.Cu") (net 6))
 (segment (start 128.8425 97.62) (end 130.44 99.2175) (width 0.2) (layer "F.Cu") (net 6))
 (segment (start 130.44 99.2175) (end 130.44 99.23) (width 0.2) (layer "F.Cu") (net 6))
 (segment (start 133.52 99.23) (end 135.89 101.6) (width 0.2) (layer "F.Cu") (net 6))
 (via (at 130.44 99.23) (size 0.6) (drill 0.3) (layers "F.Cu" "B.Cu") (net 6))
 (via (at 132.56 99.23) (size 0.6) (drill 0.3) (layers "F.Cu" "B.Cu") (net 6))
 (segment (start 130.44 99.23) (end 132.56 99.23) (width 0.2) (layer "B.Cu") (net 6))
 (segment (start 131.52 92.02) (end 132.91 93.41) (width 0.2) (layer "F.Cu") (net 9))
 (segment (start 132.91 96.08) (end 135.89 99.06) (width 0.2) (layer "F.Cu") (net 9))
 (segment (start 124.775 92.02) (end 131.52 92.02) (width 0.2) (layer "F.Cu") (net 9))
 (segment (start 132.91 93.41) (end 132.91 96.08) (width 0.2) (layer "F.Cu") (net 9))
 (segment (start 123.015 93.78) (end 124.775 92.02) (width 0.2) (layer "F.Cu") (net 9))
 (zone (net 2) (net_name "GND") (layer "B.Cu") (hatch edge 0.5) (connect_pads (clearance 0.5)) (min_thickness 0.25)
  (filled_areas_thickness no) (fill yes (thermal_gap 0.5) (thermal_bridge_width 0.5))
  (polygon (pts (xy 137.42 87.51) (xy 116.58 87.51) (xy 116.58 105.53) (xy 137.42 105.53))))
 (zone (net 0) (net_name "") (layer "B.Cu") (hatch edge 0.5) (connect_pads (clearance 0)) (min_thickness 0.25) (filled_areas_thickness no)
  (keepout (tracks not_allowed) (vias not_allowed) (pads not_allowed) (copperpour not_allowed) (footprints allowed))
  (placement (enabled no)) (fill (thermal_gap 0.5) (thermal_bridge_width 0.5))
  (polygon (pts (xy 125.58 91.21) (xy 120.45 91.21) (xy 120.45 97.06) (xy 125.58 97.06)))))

